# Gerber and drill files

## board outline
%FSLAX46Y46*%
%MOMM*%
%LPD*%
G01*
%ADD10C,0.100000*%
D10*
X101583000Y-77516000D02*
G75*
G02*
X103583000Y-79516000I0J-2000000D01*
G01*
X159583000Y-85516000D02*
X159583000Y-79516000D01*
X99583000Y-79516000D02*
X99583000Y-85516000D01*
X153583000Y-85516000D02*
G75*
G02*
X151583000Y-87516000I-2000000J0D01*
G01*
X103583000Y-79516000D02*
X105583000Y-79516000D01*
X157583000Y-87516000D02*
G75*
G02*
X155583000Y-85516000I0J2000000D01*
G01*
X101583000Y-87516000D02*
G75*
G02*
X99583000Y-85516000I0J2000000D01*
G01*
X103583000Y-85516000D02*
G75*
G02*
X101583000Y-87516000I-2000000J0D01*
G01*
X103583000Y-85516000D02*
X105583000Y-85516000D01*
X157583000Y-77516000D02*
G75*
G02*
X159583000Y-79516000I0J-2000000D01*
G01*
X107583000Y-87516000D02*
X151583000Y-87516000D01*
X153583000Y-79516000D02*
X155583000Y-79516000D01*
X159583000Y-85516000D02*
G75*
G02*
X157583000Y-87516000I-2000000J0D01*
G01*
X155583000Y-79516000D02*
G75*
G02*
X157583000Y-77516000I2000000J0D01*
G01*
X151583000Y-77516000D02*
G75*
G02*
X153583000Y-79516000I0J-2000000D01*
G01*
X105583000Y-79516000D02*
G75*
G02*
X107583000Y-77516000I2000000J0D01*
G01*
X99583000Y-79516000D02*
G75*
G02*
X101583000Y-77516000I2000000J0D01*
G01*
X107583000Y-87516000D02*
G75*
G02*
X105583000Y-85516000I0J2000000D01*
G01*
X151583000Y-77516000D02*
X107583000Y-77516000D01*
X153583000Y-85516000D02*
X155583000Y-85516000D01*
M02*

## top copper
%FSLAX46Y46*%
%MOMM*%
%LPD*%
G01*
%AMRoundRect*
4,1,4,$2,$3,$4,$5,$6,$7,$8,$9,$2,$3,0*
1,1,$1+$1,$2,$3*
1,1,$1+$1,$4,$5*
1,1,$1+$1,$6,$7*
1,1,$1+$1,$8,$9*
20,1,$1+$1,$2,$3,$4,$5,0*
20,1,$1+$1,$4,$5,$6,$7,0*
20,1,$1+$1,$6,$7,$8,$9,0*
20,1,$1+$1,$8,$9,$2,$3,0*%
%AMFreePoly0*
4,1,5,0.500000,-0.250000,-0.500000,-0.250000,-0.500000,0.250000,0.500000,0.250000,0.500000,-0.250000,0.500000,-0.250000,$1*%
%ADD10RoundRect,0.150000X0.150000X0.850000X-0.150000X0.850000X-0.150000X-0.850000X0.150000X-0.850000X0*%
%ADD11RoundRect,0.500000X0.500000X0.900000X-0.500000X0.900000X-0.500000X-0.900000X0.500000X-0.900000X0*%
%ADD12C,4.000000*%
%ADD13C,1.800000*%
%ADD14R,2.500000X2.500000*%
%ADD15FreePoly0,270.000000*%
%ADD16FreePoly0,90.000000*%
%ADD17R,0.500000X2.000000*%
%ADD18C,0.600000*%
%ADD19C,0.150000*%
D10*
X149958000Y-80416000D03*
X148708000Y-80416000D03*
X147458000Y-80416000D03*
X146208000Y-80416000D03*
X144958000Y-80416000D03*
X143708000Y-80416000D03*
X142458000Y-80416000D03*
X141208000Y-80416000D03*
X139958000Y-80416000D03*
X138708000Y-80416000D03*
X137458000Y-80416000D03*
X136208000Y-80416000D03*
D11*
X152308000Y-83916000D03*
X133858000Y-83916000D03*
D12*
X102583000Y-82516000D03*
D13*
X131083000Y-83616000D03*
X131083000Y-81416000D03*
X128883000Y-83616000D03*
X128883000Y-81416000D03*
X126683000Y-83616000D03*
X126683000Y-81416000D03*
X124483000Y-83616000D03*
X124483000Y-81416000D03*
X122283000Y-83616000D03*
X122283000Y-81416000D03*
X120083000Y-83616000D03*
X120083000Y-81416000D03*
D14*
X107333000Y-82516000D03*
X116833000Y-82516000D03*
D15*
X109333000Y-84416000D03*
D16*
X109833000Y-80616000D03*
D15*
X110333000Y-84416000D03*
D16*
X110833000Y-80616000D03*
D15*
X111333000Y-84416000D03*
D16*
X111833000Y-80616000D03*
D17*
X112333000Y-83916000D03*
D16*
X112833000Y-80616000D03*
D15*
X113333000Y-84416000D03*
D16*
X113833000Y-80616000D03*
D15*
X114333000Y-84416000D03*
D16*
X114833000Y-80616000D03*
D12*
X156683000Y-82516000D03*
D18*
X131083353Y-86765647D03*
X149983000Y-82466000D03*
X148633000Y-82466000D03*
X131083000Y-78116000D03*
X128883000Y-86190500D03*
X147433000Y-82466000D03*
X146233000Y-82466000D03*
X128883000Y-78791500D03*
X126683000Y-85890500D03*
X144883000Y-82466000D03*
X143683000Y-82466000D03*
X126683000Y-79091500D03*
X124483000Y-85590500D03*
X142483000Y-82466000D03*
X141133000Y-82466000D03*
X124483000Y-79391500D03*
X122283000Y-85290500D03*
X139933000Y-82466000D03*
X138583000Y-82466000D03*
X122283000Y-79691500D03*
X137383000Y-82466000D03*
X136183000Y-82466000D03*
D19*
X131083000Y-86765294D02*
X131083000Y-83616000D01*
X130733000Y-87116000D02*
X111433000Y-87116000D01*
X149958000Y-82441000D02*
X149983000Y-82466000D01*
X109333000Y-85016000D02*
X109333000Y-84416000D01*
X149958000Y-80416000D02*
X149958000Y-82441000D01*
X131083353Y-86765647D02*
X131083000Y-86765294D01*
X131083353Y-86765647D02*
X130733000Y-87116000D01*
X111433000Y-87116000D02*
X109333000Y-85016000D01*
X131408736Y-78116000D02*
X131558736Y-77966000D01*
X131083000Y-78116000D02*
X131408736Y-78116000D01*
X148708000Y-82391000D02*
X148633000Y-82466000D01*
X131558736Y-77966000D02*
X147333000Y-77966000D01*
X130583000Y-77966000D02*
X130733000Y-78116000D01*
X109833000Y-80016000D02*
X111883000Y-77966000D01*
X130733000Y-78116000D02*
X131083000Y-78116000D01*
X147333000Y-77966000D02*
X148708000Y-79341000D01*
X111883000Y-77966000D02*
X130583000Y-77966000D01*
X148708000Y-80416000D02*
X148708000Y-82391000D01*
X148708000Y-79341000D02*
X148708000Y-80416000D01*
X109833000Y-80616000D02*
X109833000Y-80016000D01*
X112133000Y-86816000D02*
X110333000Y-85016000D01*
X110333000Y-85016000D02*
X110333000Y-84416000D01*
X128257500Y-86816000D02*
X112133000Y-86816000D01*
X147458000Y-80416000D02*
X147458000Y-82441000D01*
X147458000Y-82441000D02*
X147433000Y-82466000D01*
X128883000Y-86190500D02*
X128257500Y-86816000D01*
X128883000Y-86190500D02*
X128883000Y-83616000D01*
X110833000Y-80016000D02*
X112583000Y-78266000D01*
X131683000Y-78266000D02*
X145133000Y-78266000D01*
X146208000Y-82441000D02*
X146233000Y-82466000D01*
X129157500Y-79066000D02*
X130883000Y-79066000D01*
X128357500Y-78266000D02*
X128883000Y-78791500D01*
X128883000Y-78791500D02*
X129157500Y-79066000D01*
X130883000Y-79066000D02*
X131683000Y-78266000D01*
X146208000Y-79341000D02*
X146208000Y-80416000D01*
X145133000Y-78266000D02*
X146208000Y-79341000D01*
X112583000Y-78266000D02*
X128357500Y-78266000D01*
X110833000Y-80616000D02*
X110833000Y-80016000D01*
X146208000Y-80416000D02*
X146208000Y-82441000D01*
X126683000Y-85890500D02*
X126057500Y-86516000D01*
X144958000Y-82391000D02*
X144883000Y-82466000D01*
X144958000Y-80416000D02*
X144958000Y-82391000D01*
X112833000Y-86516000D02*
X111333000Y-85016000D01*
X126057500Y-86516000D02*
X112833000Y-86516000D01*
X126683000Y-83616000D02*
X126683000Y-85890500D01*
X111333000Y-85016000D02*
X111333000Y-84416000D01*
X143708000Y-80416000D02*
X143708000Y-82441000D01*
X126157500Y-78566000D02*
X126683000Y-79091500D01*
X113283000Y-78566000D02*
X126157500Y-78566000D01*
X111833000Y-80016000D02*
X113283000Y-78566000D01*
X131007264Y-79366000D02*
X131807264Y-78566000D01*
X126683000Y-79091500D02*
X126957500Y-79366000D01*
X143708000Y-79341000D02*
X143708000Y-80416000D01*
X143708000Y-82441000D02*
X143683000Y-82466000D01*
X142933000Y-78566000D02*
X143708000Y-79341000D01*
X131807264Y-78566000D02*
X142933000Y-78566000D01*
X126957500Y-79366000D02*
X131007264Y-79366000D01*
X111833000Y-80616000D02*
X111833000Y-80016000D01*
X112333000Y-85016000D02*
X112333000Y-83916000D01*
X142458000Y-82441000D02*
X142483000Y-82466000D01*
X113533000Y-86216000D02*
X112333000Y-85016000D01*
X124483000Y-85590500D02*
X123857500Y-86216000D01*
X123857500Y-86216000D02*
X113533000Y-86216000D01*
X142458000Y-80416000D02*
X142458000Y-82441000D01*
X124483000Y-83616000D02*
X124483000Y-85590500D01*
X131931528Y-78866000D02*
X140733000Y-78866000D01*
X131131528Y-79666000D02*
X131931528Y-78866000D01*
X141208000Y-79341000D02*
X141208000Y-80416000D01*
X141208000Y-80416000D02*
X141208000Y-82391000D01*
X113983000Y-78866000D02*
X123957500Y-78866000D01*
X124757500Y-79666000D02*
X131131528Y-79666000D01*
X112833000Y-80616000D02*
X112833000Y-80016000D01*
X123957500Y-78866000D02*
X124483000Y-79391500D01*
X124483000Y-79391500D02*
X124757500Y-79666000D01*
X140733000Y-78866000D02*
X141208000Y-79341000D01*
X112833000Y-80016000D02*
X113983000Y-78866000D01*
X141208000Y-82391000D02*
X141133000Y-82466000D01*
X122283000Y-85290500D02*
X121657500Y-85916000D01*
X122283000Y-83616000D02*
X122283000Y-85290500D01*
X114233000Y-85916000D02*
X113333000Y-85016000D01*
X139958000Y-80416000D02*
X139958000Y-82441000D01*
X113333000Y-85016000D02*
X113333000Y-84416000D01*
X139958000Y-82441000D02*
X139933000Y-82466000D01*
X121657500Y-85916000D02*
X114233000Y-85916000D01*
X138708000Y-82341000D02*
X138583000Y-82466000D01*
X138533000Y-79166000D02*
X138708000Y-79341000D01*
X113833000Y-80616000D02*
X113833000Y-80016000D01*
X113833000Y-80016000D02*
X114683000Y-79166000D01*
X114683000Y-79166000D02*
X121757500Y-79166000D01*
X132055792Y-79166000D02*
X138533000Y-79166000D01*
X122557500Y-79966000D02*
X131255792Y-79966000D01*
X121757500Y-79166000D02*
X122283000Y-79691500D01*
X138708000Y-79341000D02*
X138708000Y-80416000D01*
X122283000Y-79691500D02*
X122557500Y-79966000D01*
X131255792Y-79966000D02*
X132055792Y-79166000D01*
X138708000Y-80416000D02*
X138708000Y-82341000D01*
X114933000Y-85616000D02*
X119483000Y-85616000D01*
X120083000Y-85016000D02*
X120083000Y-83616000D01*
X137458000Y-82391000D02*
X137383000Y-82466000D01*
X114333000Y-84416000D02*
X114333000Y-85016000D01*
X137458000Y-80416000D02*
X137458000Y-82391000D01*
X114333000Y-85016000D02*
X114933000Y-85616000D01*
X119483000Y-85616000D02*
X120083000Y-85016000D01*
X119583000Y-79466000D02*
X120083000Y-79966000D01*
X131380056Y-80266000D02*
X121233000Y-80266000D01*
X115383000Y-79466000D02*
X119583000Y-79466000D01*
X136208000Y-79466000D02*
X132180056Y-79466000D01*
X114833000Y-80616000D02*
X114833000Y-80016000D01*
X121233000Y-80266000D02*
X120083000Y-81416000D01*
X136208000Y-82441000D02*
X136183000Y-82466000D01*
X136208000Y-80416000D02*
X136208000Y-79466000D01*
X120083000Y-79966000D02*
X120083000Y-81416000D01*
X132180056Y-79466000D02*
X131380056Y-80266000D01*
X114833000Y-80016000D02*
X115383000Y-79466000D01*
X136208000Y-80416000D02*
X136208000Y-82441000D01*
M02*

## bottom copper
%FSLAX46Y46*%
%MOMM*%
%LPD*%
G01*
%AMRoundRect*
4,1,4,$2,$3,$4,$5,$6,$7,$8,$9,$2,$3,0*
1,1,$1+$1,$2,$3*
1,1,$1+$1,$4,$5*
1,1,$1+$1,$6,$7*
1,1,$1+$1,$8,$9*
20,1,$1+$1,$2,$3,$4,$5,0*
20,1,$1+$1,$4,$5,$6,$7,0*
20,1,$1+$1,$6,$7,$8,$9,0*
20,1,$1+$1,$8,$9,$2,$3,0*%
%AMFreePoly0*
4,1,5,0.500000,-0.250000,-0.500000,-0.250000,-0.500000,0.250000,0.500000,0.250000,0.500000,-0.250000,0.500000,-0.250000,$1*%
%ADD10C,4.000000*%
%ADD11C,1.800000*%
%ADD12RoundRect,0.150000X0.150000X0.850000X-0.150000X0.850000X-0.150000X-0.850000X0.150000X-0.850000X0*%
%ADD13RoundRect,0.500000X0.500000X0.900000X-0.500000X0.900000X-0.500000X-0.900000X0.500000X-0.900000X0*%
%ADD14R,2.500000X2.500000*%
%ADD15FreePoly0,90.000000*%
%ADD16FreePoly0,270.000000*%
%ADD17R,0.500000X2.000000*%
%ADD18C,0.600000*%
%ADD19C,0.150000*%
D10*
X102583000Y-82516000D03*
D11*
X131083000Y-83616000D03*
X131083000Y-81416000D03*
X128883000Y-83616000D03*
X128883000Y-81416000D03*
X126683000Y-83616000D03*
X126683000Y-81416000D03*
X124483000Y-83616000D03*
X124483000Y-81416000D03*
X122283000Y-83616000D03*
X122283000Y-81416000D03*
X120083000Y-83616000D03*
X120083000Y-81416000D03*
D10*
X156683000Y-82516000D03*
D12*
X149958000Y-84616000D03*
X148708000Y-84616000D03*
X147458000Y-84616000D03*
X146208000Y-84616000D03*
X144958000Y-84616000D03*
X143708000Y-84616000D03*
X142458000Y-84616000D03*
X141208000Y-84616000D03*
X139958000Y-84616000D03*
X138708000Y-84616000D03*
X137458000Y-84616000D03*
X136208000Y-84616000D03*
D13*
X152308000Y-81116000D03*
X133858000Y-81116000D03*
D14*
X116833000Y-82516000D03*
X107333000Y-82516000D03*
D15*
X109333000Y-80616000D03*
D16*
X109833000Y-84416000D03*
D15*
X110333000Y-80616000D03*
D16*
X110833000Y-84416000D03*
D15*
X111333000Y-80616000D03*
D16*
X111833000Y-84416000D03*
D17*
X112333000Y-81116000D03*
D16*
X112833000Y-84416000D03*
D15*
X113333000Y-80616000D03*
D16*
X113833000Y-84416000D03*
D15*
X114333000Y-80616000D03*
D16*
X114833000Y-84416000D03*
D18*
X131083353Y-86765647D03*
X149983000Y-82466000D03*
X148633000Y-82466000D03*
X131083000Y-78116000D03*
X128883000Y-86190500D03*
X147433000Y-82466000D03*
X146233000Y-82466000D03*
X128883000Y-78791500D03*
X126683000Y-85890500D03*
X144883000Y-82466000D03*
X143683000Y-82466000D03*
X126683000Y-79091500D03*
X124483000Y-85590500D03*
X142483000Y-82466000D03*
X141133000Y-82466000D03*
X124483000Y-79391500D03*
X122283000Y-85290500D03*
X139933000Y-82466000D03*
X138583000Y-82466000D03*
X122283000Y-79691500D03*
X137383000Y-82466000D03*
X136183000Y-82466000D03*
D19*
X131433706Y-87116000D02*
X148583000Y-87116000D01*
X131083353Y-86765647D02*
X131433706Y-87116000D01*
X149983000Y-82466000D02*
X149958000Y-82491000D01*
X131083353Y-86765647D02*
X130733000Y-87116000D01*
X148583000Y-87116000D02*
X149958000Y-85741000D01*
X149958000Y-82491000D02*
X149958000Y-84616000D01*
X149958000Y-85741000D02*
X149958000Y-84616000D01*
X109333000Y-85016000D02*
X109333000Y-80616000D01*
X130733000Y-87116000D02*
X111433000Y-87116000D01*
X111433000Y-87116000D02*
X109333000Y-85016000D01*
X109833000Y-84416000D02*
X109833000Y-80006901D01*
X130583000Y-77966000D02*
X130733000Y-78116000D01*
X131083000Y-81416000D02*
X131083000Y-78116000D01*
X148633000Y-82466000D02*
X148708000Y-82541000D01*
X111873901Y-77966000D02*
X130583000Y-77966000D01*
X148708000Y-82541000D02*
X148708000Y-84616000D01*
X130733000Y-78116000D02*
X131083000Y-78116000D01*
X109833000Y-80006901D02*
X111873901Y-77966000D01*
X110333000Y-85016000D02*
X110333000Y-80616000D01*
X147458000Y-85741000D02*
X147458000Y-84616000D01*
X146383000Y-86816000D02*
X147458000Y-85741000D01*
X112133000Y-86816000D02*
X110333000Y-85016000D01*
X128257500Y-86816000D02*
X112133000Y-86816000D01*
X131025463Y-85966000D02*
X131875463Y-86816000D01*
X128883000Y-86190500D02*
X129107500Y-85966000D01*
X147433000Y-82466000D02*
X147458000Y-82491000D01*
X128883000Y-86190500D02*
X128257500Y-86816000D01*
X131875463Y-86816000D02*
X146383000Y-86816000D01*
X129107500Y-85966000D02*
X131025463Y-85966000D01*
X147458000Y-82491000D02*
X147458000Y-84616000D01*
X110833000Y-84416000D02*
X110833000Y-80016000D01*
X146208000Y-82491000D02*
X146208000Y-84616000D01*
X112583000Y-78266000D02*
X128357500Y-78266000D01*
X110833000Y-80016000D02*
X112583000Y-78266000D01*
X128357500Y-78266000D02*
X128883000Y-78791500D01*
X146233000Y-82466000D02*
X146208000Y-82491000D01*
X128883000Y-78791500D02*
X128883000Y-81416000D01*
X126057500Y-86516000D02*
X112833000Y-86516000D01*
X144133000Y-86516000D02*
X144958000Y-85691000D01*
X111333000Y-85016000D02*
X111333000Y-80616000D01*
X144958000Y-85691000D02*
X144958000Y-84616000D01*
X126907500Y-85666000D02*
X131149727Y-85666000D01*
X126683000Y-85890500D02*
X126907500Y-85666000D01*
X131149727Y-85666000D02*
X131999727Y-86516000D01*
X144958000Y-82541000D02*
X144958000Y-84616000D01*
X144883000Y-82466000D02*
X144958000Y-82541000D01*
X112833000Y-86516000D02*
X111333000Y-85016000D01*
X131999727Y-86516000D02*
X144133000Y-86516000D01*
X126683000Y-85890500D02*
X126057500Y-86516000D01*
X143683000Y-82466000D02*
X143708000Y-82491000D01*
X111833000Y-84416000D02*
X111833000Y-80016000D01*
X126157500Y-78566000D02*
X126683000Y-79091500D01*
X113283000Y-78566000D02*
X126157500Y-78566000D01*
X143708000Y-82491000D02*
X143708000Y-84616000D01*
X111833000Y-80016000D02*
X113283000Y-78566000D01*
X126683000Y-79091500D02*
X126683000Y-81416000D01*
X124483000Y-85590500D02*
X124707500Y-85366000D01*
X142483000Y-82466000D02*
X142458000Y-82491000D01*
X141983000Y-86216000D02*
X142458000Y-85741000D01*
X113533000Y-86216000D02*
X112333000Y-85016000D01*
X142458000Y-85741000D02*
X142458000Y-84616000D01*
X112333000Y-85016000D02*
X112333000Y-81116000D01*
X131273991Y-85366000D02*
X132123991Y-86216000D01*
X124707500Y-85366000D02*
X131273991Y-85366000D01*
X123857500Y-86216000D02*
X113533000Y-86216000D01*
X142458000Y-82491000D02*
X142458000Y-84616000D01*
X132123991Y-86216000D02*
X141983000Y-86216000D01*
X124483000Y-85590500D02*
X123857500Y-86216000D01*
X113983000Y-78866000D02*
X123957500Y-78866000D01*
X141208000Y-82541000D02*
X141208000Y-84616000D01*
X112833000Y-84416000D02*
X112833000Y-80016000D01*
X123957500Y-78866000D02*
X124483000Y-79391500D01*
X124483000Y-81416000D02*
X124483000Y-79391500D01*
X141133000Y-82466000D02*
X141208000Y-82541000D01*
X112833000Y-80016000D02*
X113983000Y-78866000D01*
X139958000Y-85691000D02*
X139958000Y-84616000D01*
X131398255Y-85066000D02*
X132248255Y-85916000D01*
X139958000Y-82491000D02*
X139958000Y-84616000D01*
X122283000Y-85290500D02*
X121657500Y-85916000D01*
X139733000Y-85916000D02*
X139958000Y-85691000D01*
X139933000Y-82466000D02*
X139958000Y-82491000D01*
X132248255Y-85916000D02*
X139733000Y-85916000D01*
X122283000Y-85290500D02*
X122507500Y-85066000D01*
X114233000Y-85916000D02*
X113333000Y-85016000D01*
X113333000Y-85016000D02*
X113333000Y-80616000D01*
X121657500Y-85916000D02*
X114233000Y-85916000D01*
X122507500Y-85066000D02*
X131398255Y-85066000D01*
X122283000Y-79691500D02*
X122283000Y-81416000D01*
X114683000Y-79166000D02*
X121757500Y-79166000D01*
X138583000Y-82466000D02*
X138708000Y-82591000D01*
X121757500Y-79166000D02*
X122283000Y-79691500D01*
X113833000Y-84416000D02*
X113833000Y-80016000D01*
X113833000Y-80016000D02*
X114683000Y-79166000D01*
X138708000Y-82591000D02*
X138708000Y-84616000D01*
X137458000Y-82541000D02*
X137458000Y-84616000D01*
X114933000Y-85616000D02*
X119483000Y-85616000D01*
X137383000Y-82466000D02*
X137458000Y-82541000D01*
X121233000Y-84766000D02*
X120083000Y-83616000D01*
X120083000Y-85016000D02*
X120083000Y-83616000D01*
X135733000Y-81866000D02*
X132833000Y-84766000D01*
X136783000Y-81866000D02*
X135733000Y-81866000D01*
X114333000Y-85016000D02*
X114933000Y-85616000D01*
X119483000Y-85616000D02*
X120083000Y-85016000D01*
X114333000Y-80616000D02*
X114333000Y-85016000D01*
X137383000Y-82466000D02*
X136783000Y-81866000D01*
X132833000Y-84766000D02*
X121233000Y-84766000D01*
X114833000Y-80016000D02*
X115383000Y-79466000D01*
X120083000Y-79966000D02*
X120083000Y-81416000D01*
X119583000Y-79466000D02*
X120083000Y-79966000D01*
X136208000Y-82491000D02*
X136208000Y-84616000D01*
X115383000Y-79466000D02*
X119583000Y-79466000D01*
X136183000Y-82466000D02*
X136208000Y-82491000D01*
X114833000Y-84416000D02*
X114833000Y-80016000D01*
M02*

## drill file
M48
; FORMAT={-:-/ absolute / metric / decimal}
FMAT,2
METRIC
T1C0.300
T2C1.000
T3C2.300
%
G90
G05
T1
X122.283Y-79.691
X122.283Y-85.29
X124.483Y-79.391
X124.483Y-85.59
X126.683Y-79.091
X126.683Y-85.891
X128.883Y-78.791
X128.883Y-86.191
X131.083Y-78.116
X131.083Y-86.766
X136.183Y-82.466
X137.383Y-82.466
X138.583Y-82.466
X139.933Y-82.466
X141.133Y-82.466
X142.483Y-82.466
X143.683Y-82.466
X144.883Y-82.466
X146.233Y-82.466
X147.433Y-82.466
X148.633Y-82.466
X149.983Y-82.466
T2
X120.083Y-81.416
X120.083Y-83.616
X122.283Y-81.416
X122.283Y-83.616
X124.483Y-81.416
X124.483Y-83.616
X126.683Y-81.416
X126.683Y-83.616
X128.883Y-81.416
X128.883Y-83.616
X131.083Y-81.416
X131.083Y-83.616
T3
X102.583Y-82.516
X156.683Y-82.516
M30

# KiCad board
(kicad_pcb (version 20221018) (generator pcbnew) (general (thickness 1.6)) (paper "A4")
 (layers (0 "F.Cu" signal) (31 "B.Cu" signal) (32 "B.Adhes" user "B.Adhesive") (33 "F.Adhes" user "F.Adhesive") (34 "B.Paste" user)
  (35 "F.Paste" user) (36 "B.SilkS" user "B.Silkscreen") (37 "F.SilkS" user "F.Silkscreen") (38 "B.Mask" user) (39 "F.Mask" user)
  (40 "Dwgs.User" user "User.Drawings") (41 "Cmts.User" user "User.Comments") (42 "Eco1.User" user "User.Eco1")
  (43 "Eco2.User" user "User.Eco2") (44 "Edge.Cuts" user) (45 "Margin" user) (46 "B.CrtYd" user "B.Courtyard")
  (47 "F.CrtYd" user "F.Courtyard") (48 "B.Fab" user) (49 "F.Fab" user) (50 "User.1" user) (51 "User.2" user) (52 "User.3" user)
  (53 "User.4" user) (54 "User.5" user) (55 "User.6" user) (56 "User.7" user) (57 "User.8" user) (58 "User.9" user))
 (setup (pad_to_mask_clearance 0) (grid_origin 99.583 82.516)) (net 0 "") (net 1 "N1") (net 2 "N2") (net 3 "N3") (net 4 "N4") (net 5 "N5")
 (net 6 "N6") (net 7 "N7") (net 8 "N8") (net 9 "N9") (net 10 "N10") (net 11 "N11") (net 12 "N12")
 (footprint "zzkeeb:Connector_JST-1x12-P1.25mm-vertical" (layer "F.Cu") (at 143.083 82.516 180)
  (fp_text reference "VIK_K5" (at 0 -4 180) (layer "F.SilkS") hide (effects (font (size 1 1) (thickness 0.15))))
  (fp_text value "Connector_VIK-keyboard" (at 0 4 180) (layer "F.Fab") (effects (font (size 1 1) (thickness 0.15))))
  (pad "1" smd roundrect (at -6.875 2.1 180) (size 0.6 2) (layers "F.Cu" "F.Paste" "F.Mask") (roundrect_rratio 0.25) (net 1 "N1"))
  (pad "2" smd roundrect (at -5.625 2.1 180) (size 0.6 2) (layers "F.Cu" "F.Paste" "F.Mask") (roundrect_rratio 0.25) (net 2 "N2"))
  (pad "3" smd roundrect (at -4.375 2.1 180) (size 0.6 2) (layers "F.Cu" "F.Paste" "F.Mask") (roundrect_rratio 0.25) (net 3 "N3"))
  (pad "4" smd roundrect (at -3.125 2.1 180) (size 0.6 2) (layers "F.Cu" "F.Paste" "F.Mask") (roundrect_rratio 0.25) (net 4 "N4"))
  (pad "5" smd roundrect (at -1.875 2.1 180) (size 0.6 2) (layers "F.Cu" "F.Paste" "F.Mask") (roundrect_rratio 0.25) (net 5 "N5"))
  (pad "6" smd roundrect (at -0.625 2.1 180) (size 0.6 2) (layers "F.Cu" "F.Paste" "F.Mask") (roundrect_rratio 0.25) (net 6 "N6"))
  (pad "7" smd roundrect (at 0.625 2.1 180) (size 0.6 2) (layers "F.Cu" "F.Paste" "F.Mask") (roundrect_rratio 0.25) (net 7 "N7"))
  (pad "8" smd roundrect (at 1.875 2.1 180) (size 0.6 2) (layers "F.Cu" "F.Paste" "F.Mask") (roundrect_rratio 0.25) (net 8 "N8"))
  (pad "9" smd roundrect (at 3.125 2.1 180) (size 0.6 2) (layers "F.Cu" "F.Paste" "F.Mask") (roundrect_rratio 0.25) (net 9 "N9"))
  (pad "10" smd roundrect (at 4.375 2.1 180) (size 0.6 2) (layers "F.Cu" "F.Paste" "F.Mask") (roundrect_rratio 0.25) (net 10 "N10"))
  (pad "11" smd roundrect (at 5.625 2.1 180) (size 0.6 2) (layers "F.Cu" "F.Paste" "F.Mask") (roundrect_rratio 0.25) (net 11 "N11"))
  (pad "12" smd roundrect (at 6.875 2.1 180) (size 0.6 2) (layers "F.Cu" "F.Paste" "F.Mask") (roundrect_rratio 0.25) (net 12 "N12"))
  (pad "MP" smd roundrect (at -9.225 -1.4 180) (size 2 2.8) (layers "F.Cu" "F.Paste" "F.Mask") (roundrect_rratio 0.25))
  (pad "MP" smd roundrect (at 9.225 -1.4 180) (size 2 2.8) (layers "F.Cu" "F.Paste" "F.Mask") (roundrect_rratio 0.25)))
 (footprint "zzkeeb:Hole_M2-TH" (layer "F.Cu") (at 102.583 82.516)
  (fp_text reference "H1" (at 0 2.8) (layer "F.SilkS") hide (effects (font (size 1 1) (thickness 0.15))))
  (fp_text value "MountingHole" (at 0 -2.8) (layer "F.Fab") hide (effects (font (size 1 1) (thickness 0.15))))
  (pad "" thru_hole circle (at 0 0) (size 4 4) (drill 2.3) (layers "*.Cu" "*.Mask")))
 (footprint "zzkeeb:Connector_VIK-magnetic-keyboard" (layer "F.Cu") (at 125.583 82.516 90)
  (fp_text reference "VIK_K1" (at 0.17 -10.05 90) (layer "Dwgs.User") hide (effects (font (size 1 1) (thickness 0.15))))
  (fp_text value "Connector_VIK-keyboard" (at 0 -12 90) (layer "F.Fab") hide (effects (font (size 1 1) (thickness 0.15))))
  (pad "1" thru_hole circle (at -1.1 5.5 270) (size 1.8 1.8) (drill 1) (layers "*.Cu" "*.Mask") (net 1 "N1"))
  (pad "2" thru_hole circle (at 1.1 5.5 270) (size 1.8 1.8) (drill 1) (layers "*.Cu" "*.Mask") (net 2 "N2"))
  (pad "3" thru_hole circle (at -1.1 3.3 270) (size 1.8 1.8) (drill 1) (layers "*.Cu" "*.Mask") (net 3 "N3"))
  (pad "4" thru_hole circle (at 1.1 3.3 270) (size 1.8 1.8) (drill 1) (layers "*.Cu" "*.Mask") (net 4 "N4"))
  (pad "5" thru_hole circle (at -1.1 1.1 270) (size 1.8 1.8) (drill 1) (layers "*.Cu" "*.Mask") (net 5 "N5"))
  (pad "6" thru_hole circle (at 1.1 1.1 270) (size 1.8 1.8) (drill 1) (layers "*.Cu" "*.Mask") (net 6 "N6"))
  (pad "7" thru_hole circle (at -1.1 -1.1 270) (size 1.8 1.8) (drill 1) (layers "*.Cu" "*.Mask") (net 7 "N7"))
  (pad "8" thru_hole circle (at 1.1 -1.1 270) (size 1.8 1.8) (drill 1) (layers "*.Cu" "*.Mask") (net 8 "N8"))
  (pad "9" thru_hole circle (at -1.1 -3.3 270) (size 1.8 1.8) (drill 1) (layers "*.Cu" "*.Mask") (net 9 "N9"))
  (pad "10" thru_hole circle (at 1.1 -3.3 270) (size 1.8 1.8) (drill 1) (layers "*.Cu" "*.Mask") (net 10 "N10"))
  (pad "11" thru_hole circle (at -1.1 -5.5 270) (size 1.8 1.8) (drill 1) (layers "*.Cu" "*.Mask") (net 11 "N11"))
  (pad "12" thru_hole circle (at 1.1 -5.5 270) (size 1.8 1.8) (drill 1) (layers "*.Cu" "*.Mask") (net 12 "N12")))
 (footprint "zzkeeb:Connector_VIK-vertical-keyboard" (layer "F.Cu") (at 112.083 82.516 90)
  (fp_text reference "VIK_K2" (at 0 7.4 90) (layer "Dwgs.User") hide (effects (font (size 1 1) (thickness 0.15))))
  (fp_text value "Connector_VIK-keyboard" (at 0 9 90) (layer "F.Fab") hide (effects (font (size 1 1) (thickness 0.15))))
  (pad "" smd rect (at 0 -4.75 90) (size 2.5 2.5) (layers "F.Cu" "F.Paste" "F.Mask"))
  (pad "" smd rect (at 0 4.75 90) (size 2.5 2.5) (layers "F.Cu" "F.Paste" "F.Mask"))
  (pad "1" smd custom (at -1.9 -2.75 270) (size 1 0.5) (layers "F.Cu" "F.Paste" "F.Mask") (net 1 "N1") (thermal_bridge_angle 45)
   (options (clearance outline) (anchor rect)) (primitives))
  (pad "2" smd custom (at 1.9 -2.25 90) (size 1 0.5) (layers "F.Cu" "F.Paste" "F.Mask") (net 2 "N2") (thermal_bridge_angle 45)
   (options (clearance outline) (anchor rect)) (primitives))
  (pad "3" smd custom (at -1.9 -1.75 270) (size 1 0.5) (layers "F.Cu" "F.Paste" "F.Mask") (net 3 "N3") (thermal_bridge_angle 45)
   (options (clearance outline) (anchor rect)) (primitives))
  (pad "4" smd custom (at 1.9 -1.25 90) (size 1 0.5) (layers "F.Cu" "F.Paste" "F.Mask") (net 4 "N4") (thermal_bridge_angle 45)
   (options (clearance outline) (anchor rect)) (primitives))
  (pad "5" smd custom (at -1.9 -0.75 270) (size 1 0.5) (layers "F.Cu" "F.Paste" "F.Mask") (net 5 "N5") (thermal_bridge_angle 45)
   (options (clearance outline) (anchor rect)) (primitives))
  (pad "6" smd custom (at 1.9 -0.25 90) (size 1 0.5) (layers "F.Cu" "F.Paste" "F.Mask") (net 6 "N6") (thermal_bridge_angle 45)
   (options (clearance outline) (anchor rect)) (primitives))
  (pad "7" smd rect (at -1.4 0.25) (size 0.5 2) (layers "F.Cu" "F.Paste" "F.Mask") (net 7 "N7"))
  (pad "8" smd custom (at 1.9 0.75 90) (size 1 0.5) (layers "F.Cu" "F.Paste" "F.Mask") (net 8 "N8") (thermal_bridge_angle 45)
   (options (clearance outline) (anchor rect)) (primitives))
  (pad "9" smd custom (at -1.9 1.25 270) (size 1 0.5) (layers "F.Cu" "F.Paste" "F.Mask") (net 9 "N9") (thermal_bridge_angle 45)
   (options (clearance outline) (anchor rect)) (primitives))
  (pad "10" smd custom (at 1.9 1.75 90) (size 1 0.5) (layers "F.Cu" "F.Paste" "F.Mask") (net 10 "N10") (thermal_bridge_angle 45)
   (options (clearance outline) (anchor rect)) (primitives))
  (pad "11" smd custom (at -1.9 2.25 270) (size 1 0.5) (layers "F.Cu" "F.Paste" "F.Mask") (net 11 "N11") (thermal_bridge_angle 45)
   (options (clearance outline) (anchor rect)) (primitives))
  (pad "12" smd custom (at 1.9 2.75 90) (size 1 0.5) (layers "F.Cu" "F.Paste" "F.Mask") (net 12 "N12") (thermal_bridge_angle 45)
   (options (clearance outline) (anchor rect)) (primitives)))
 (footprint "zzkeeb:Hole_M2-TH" (layer "F.Cu") (at 156.683 82.516)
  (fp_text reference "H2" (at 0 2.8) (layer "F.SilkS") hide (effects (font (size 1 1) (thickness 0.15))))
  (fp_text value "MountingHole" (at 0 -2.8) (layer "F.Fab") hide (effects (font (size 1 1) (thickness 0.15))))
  (pad "" thru_hole circle (at 0 0) (size 4 4) (drill 2.3) (layers "*.Cu" "*.Mask")))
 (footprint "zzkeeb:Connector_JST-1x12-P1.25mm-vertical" (layer "B.Cu") (at 143.083 82.516 180)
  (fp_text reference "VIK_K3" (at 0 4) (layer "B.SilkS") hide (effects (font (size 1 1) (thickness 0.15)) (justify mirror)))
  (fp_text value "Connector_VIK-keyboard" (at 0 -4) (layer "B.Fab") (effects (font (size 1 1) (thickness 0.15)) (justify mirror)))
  (pad "1" smd roundrect (at -6.875 -2.1 180) (size 0.6 2) (layers "B.Cu" "B.Paste" "B.Mask") (roundrect_rratio 0.25) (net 1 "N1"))
  (pad "2" smd roundrect (at -5.625 -2.1 180) (size 0.6 2) (layers "B.Cu" "B.Paste" "B.Mask") (roundrect_rratio 0.25) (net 2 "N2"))
  (pad "3" smd roundrect (at -4.375 -2.1 180) (size 0.6 2) (layers "B.Cu" "B.Paste" "B.Mask") (roundrect_rratio 0.25) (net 3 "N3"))
  (pad "4" smd roundrect (at -3.125 -2.1 180) (size 0.6 2) (layers "B.Cu" "B.Paste" "B.Mask") (roundrect_rratio 0.25) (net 4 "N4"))
  (pad "5" smd roundrect (at -1.875 -2.1 180) (size 0.6 2) (layers "B.Cu" "B.Paste" "B.Mask") (roundrect_rratio 0.25) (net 5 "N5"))
  (pad "6" smd roundrect (at -0.625 -2.1 180) (size 0.6 2) (layers "B.Cu" "B.Paste" "B.Mask") (roundrect_rratio 0.25) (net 6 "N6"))
  (pad "7" smd roundrect (at 0.625 -2.1 180) (size 0.6 2) (layers "B.Cu" "B.Paste" "B.Mask") (roundrect_rratio 0.25) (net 7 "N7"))
  (pad "8" smd roundrect (at 1.875 -2.1 180) (size 0.6 2) (layers "B.Cu" "B.Paste" "B.Mask") (roundrect_rratio 0.25) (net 8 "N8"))
  (pad "9" smd roundrect (at 3.125 -2.1 180) (size 0.6 2) (layers "B.Cu" "B.Paste" "B.Mask") (roundrect_rratio 0.25) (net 9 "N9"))
  (pad "10" smd roundrect (at 4.375 -2.1 180) (size 0.6 2) (layers "B.Cu" "B.Paste" "B.Mask") (roundrect_rratio 0.25) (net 10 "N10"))
  (pad "11" smd roundrect (at 5.625 -2.1 180) (size 0.6 2) (layers "B.Cu" "B.Paste" "B.Mask") (roundrect_rratio 0.25) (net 11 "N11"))
  (pad "12" smd roundrect (at 6.875 -2.1 180) (size 0.6 2) (layers "B.Cu" "B.Paste" "B.Mask") (roundrect_rratio 0.25) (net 12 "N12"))
  (pad "MP" smd roundrect (at -9.225 1.4 180) (size 2 2.8) (layers "B.Cu" "B.Paste" "B.Mask") (roundrect_rratio 0.25))
  (pad "MP" smd roundrect (at 9.225 1.4 180) (size 2 2.8) (layers "B.Cu" "B.Paste" "B.Mask") (roundrect_rratio 0.25)))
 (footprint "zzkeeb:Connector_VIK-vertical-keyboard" (layer "B.Cu") (at 112.083 82.516 -90)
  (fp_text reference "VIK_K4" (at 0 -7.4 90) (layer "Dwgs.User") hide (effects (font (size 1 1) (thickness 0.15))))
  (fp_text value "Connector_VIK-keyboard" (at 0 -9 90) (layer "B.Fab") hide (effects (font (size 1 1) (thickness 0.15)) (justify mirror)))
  (pad "" smd rect (at 0 -4.75 270) (size 2.5 2.5) (layers "B.Cu" "B.Paste" "B.Mask"))
  (pad "" smd rect (at 0 4.75 270) (size 2.5 2.5) (layers "B.Cu" "B.Paste" "B.Mask"))
  (pad "1" smd custom (at -1.9 2.75 90) (size 1 0.5) (layers "B.Cu" "B.Paste" "B.Mask") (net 1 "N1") (thermal_bridge_angle 45)
   (options (clearance outline) (anchor rect)) (primitives))
  (pad "2" smd custom (at 1.9 2.25 270) (size 1 0.5) (layers "B.Cu" "B.Paste" "B.Mask") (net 2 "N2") (thermal_bridge_angle 45)
   (options (clearance outline) (anchor rect)) (primitives))
  (pad "3" smd custom (at -1.9 1.75 90) (size 1 0.5) (layers "B.Cu" "B.Paste" "B.Mask") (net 3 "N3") (thermal_bridge_angle 45)
   (options (clearance outline) (anchor rect)) (primitives))
  (pad "4" smd custom (at 1.9 1.25 270) (size 1 0.5) (layers "B.Cu" "B.Paste" "B.Mask") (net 4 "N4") (thermal_bridge_angle 45)
   (options (clearance outline) (anchor rect)) (primitives))
  (pad "5" smd custom (at -1.9 0.75 90) (size 1 0.5) (layers "B.Cu" "B.Paste" "B.Mask") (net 5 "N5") (thermal_bridge_angle 45)
   (options (clearance outline) (anchor rect)) (primitives))
  (pad "6" smd custom (at 1.9 0.25 270) (size 1 0.5) (layers "B.Cu" "B.Paste" "B.Mask") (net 6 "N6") (thermal_bridge_angle 45)
   (options (clearance outline) (anchor rect)) (primitives))
  (pad "7" smd rect (at -1.4 -0.25) (size 0.5 2) (layers "B.Cu" "B.Paste" "B.Mask") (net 7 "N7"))
  (pad "8" smd custom (at 1.9 -0.75 270) (size 1 0.5) (layers "B.Cu" "B.Paste" "B.Mask") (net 8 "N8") (thermal_bridge_angle 45)
   (options (clearance outline) (anchor rect)) (primitives))
  (pad "9" smd custom (at -1.9 -1.25 90) (size 1 0.5) (layers "B.Cu" "B.Paste" "B.Mask") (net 9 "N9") (thermal_bridge_angle 45)
   (options (clearance outline) (anchor rect)) (primitives))
  (pad "10" smd custom (at 1.9 -1.75 270) (size 1 0.5) (layers "B.Cu" "B.Paste" "B.Mask") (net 10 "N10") (thermal_bridge_angle 45)
   (options (clearance outline) (anchor rect)) (primitives))
  (pad "11" smd custom (at -1.9 -2.25 90) (size 1 0.5) (layers "B.Cu" "B.Paste" "B.Mask") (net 11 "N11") (thermal_bridge_angle 45)
   (options (clearance outline) (anchor rect)) (primitives))
  (pad "12" smd custom (at 1.9 -2.75 270) (size 1 0.5) (layers "B.Cu" "B.Paste" "B.Mask") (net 12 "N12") (thermal_bridge_angle 45)
   (options (clearance outline) (anchor rect)) (primitives)))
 (gr_arc (start 101.583 77.516) (mid 102.997214 78.101786) (end 103.583 79.516) (stroke (width 0.1) (type default)) (layer "Edge.Cuts"))
 (gr_line (start 159.583 85.516) (end 159.583 79.516) (stroke (width 0.1) (type default)) (layer "Edge.Cuts"))
 (gr_line (start 99.583 79.516) (end 99.583 85.516) (stroke (width 0.1) (type default)) (layer "Edge.Cuts"))
 (gr_arc (start 153.583 85.516) (mid 152.997214 86.930214) (end 151.583 87.516) (stroke (width 0.1) (type default)) (layer "Edge.Cuts"))
 (gr_line (start 103.583 79.516) (end 105.583 79.516) (stroke (width 0.1) (type default)) (layer "Edge.Cuts"))
 (gr_arc (start 157.583 87.516) (mid 156.168786 86.930214) (end 155.583 85.516) (stroke (width 0.1) (type default)) (layer "Edge.Cuts"))
 (gr_arc (start 101.583 87.516) (mid 100.168786 86.930214) (end 99.583 85.516) (stroke (width 0.1) (type default)) (layer "Edge.Cuts"))
 (gr_arc (start 103.583 85.516) (mid 102.997214 86.930214) (end 101.583 87.516) (stroke (width 0.1) (type default)) (layer "Edge.Cuts"))
 (gr_line (start 103.583 85.516) (end 105.583 85.516) (stroke (width 0.1) (type default)) (layer "Edge.Cuts"))
 (gr_arc (start 157.583 77.516) (mid 158.997214 78.101786) (end 159.583 79.516) (stroke (width 0.1) (type default)) (layer "Edge.Cuts"))
 (gr_line (start 107.583 87.516) (end 151.583 87.516) (stroke (width 0.1) (type default)) (layer "Edge.Cuts"))
 (gr_line (start 153.583 79.516) (end 155.583 79.516) (stroke (width 0.1) (type default)) (layer "Edge.Cuts"))
 (gr_arc (start 159.583 85.516) (mid 158.997214 86.930214) (end 157.583 87.516) (stroke (width 0.1) (type default)) (layer "Edge.Cuts"))
 (gr_arc (start 155.583 79.516) (mid 156.168786 78.101786) (end 157.583 77.516) (stroke (width 0.1) (type default)) (layer "Edge.Cuts"))
 (gr_arc (start 151.583 77.516) (mid 152.997214 78.101786) (end 153.583 79.516) (stroke (width 0.1) (type default)) (layer "Edge.Cuts"))
 (gr_arc (start 105.583 79.516) (mid 106.168786 78.101786) (end 107.583 77.516) (stroke (width 0.1) (type default)) (layer "Edge.Cuts"))
 (gr_arc (start 99.583 79.516) (mid 100.168786 78.101786) (end 101.583 77.516) (stroke (width 0.1) (type default)) (layer "Edge.Cuts"))
 (gr_arc (start 107.583 87.516) (mid 106.168786 86.930214) (end 105.583 85.516) (stroke (width 0.1) (type default)) (layer "Edge.Cuts"))
 (gr_line (start 151.583 77.516) (end 107.583 77.516) (stroke (width 0.1) (type default)) (layer "Edge.Cuts"))
 (gr_line (start 153.583 85.516) (end 155.583 85.516) (stroke (width 0.1) (type default)) (layer "Edge.Cuts"))
 (segment (start 131.083 86.765294) (end 131.083 83.616) (width 0.15) (layer "F.Cu") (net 1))
 (segment (start 130.733 87.116) (end 111.433 87.116) (width 0.15) (layer "F.Cu") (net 1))
 (segment (start 149.958 82.441) (end 149.983 82.466) (width 0.15) (layer "F.Cu") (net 1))
 (segment (start 109.333 85.016) (end 109.333 84.416) (width 0.15) (layer "F.Cu") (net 1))
 (segment (start 149.958 80.416) (end 149.958 82.441) (width 0.15) (layer "F.Cu") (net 1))
 (segment (start 131.083353 86.765647) (end 131.083 86.765294) (width 0.15) (layer "F.Cu") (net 1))
 (segment (start 131.083353 86.765647) (end 130.733 87.116) (width 0.15) (layer "F.Cu") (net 1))
 (segment (start 111.433 87.116) (end 109.333 85.016) (width 0.15) (layer "F.Cu") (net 1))
 (via (at 131.083353 86.765647) (size 0.6) (drill 0.3) (layers "F.Cu" "B.Cu") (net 1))
 (via (at 149.983 82.466) (size 0.6) (drill 0.3) (layers "F.Cu" "B.Cu") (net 1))
 (segment (start 131.433706 87.116) (end 148.583 87.116) (width 0.15) (layer "B.Cu") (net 1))
 (segment (start 131.083353 86.765647) (end 131.433706 87.116) (width 0.15) (layer "B.Cu") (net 1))
 (segment (start 149.983 82.466) (end 149.958 82.491) (width 0.15) (layer "B.Cu") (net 1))
 (segment (start 131.083353 86.765647) (end 130.733 87.116) (width 0.15) (layer "B.Cu") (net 1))
 (segment (start 148.583 87.116) (end 149.958 85.741) (width 0.15) (layer "B.Cu") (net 1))
 (segment (start 149.958 82.491) (end 149.958 84.616) (width 0.15) (layer "B.Cu") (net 1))
 (segment (start 149.958 85.741) (end 149.958 84.616) (width 0.15) (layer "B.Cu") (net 1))
 (segment (start 109.333 85.016) (end 109.333 80.616) (width 0.15) (layer "B.Cu") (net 1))
 (segment (start 130.733 87.116) (end 111.433 87.116) (width 0.15) (layer "B.Cu") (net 1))
 (segment (start 111.433 87.116) (end 109.333 85.016) (width 0.15) (layer "B.Cu") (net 1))
 (segment (start 131.408736 78.116) (end 131.558736 77.966) (width 0.15) (layer "F.Cu") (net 2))
 (segment (start 131.083 78.116) (end 131.408736 78.116) (width 0.15) (layer "F.Cu") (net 2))
 (segment (start 148.708 82.391) (end 148.633 82.466) (width 0.15) (layer "F.Cu") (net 2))
 (segment (start 131.558736 77.966) (end 147.333 77.966) (width 0.15) (layer "F.Cu") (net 2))
 (segment (start 130.583 77.966) (end 130.733 78.116) (width 0.15) (layer "F.Cu") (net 2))
 (segment (start 109.833 80.016) (end 111.883 77.966) (width 0.15) (layer "F.Cu") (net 2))
 (segment (start 130.733 78.116) (end 131.083 78.116) (width 0.15) (layer "F.Cu") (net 2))
 (segment (start 147.333 77.966) (end 148.708 79.341) (width 0.15) (layer "F.Cu") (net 2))
 (segment (start 111.883 77.966) (end 130.583 77.966) (width 0.15) (layer "F.Cu") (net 2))
 (segment (start 148.708 80.416) (end 148.708 82.391) (width 0.15) (layer "F.Cu") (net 2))
 (segment (start 148.708 79.341) (end 148.708 80.416) (width 0.15) (layer "F.Cu") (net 2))
 (segment (start 109.833 80.616) (end 109.833 80.016) (width 0.15) (layer "F.Cu") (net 2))
 (via (at 148.633 82.466) (size 0.6) (drill 0.3) (layers "F.Cu" "B.Cu") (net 2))
 (via (at 131.083 78.116) (size 0.6) (drill 0.3) (layers "F.Cu" "B.Cu") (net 2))
 (segment (start 109.833 84.416) (end 109.833 80.006901) (width 0.15) (layer "B.Cu") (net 2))
 (segment (start 130.583 77.966) (end 130.733 78.116) (width 0.15) (layer "B.Cu") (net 2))
 (segment (start 131.083 81.416) (end 131.083 78.116) (width 0.15) (layer "B.Cu") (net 2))
 (segment (start 148.633 82.466) (end 148.708 82.541) (width 0.15) (layer "B.Cu") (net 2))
 (segment (start 111.873901 77.966) (end 130.583 77.966) (width 0.15) (layer "B.Cu") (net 2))
 (segment (start 148.708 82.541) (end 148.708 84.616) (width 0.15) (layer "B.Cu") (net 2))
 (segment (start 130.733 78.116) (end 131.083 78.116) (width 0.15) (layer "B.Cu") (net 2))
 (segment (start 109.833 80.006901) (end 111.873901 77.966) (width 0.15) (layer "B.Cu") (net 2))
 (segment (start 112.133 86.816) (end 110.333 85.016) (width 0.15) (layer "F.Cu") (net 3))
 (segment (start 110.333 85.016) (end 110.333 84.416) (width 0.15) (layer "F.Cu") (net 3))
 (segment (start 128.2575 86.816) (end 112.133 86.816) (width 0.15) (layer "F.Cu") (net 3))
 (segment (start 147.458 80.416) (end 147.458 82.441) (width 0.15) (layer "F.Cu") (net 3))
 (segment (start 147.458 82.441) (end 147.433 82.466) (width 0.15) (layer "F.Cu") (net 3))
 (segment (start 128.883 86.1905) (end 128.2575 86.816) (width 0.15) (layer "F.Cu") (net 3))
 (segment (start 128.883 86.1905) (end 128.883 83.616) (width 0.15) (layer "F.Cu") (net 3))
 (via (at 128.883 86.1905) (size 0.6) (drill 0.3) (layers "F.Cu" "B.Cu") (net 3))
 (via (at 147.433 82.466) (size 0.6) (drill 0.3) (layers "F.Cu" "B.Cu") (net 3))
 (segment (start 110.333 85.016) (end 110.333 80.616) (width 0.15) (layer "B.Cu") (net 3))
 (segment (start 147.458 85.741) (end 147.458 84.616) (width 0.15) (layer "B.Cu") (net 3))
 (segment (start 146.383 86.816) (end 147.458 85.741) (width 0.15) (layer "B.Cu") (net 3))
 (segment (start 112.133 86.816) (end 110.333 85.016) (width 0.15) (layer "B.Cu") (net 3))
 (segment (start 128.2575 86.816) (end 112.133 86.816) (width 0.15) (layer "B.Cu") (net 3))
 (segment (start 131.025463 85.966) (end 131.875463 86.816) (width 0.15) (layer "B.Cu") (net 3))
 (segment (start 128.883 86.1905) (end 129.1075 85.966) (width 0.15) (layer "B.Cu") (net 3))
 (segment (start 147.433 82.466) (end 147.458 82.491) (width 0.15) (layer "B.Cu") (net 3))
 (segment (start 128.883 86.1905) (end 128.2575 86.816) (width 0.15) (layer "B.Cu") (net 3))
 (segment (start 131.875463 86.816) (end 146.383 86.816) (width 0.15) (layer "B.Cu") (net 3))
 (segment (start 129.1075 85.966) (end 131.025463 85.966) (width 0.15) (layer "B.Cu") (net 3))
 (segment (start 147.458 82.491) (end 147.458 84.616) (width 0.15) (layer "B.Cu") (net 3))
 (segment (start 110.833 80.016) (end 112.583 78.266) (width 0.15) (layer "F.Cu") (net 4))
 (segment (start 131.683 78.266) (end 145.133 78.266) (width 0.15) (layer "F.Cu") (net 4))
 (segment (start 146.208 82.441) (end 146.233 82.466) (width 0.15) (layer "F.Cu") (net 4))
 (segment (start 129.1575 79.066) (end 130.883 79.066) (width 0.15) (layer "F.Cu") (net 4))
 (segment (start 128.3575 78.266) (end 128.883 78.7915) (width 0.15) (layer "F.Cu") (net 4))
 (segment (start 128.883 78.7915) (end 129.1575 79.066) (width 0.15) (layer "F.Cu") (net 4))
 (segment (start 130.883 79.066) (end 131.683 78.266) (width 0.15) (layer "F.Cu") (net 4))
 (segment (start 146.208 79.341) (end 146.208 80.416) (width 0.15) (layer "F.Cu") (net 4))
 (segment (start 145.133 78.266) (end 146.208 79.341) (width 0.15) (layer "F.Cu") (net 4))
 (segment (start 112.583 78.266) (end 128.3575 78.266) (width 0.15) (layer "F.Cu") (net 4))
 (segment (start 110.833 80.616) (end 110.833 80.016) (width 0.15) (layer "F.Cu") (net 4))
 (segment (start 146.208 80.416) (end 146.208 82.441) (width 0.15) (layer "F.Cu") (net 4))
 (via (at 146.233 82.466) (size 0.6) (drill 0.3) (layers "F.Cu" "B.Cu") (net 4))
 (via (at 128.883 78.7915) (size 0.6) (drill 0.3) (layers "F.Cu" "B.Cu") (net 4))
 (segment (start 110.833 84.416) (end 110.833 80.016) (width 0.15) (layer "B.Cu") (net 4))
 (segment (start 146.208 82.491) (end 146.208 84.616) (width 0.15) (layer "B.Cu") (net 4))
 (segment (start 112.583 78.266) (end 128.3575 78.266) (width 0.15) (layer "B.Cu") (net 4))
 (segment (start 110.833 80.016) (end 112.583 78.266) (width 0.15) (layer "B.Cu") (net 4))
 (segment (start 128.3575 78.266) (end 128.883 78.7915) (width 0.15) (layer "B.Cu") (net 4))
 (segment (start 146.233 82.466) (end 146.208 82.491) (width 0.15) (layer "B.Cu") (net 4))
 (segment (start 128.883 78.7915) (end 128.883 81.416) (width 0.15) (layer "B.Cu") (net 4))
 (segment (start 126.683 85.8905) (end 126.0575 86.516) (width 0.15) (layer "F.Cu") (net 5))
 (segment (start 144.958 82.391) (end 144.883 82.466) (width 0.15) (layer "F.Cu") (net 5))
 (segment (start 144.958 80.416) (end 144.958 82.391) (width 0.15) (layer "F.Cu") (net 5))
 (segment (start 112.833 86.516) (end 111.333 85.016) (width 0.15) (layer "F.Cu") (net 5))
 (segment (start 126.0575 86.516) (end 112.833 86.516) (width 0.15) (layer "F.Cu") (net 5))
 (segment (start 126.683 83.616) (end 126.683 85.8905) (width 0.15) (layer "F.Cu") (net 5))
 (segment (start 111.333 85.016) (end 111.333 84.416) (width 0.15) (layer "F.Cu") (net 5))
 (via (at 126.683 85.8905) (size 0.6) (drill 0.3) (layers "F.Cu" "B.Cu") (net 5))
 (via (at 144.883 82.466) (size 0.6) (drill 0.3) (layers "F.Cu" "B.Cu") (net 5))
 (segment (start 126.0575 86.516) (end 112.833 86.516) (width 0.15) (layer "B.Cu") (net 5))
 (segment (start 144.133 86.516) (end 144.958 85.691) (width 0.15) (layer "B.Cu") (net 5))
 (segment (start 111.333 85.016) (end 111.333 80.616) (width 0.15) (layer "B.Cu") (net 5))
 (segment (start 144.958 85.691) (end 144.958 84.616) (width 0.15) (layer "B.Cu") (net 5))
 (segment (start 126.9075 85.666) (end 131.149727 85.666) (width 0.15) (layer "B.Cu") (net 5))
 (segment (start 126.683 85.8905) (end 126.9075 85.666) (width 0.15) (layer "B.Cu") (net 5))
 (segment (start 131.149727 85.666) (end 131.999727 86.516) (width 0.15) (layer "B.Cu") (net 5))
 (segment (start 144.958 82.541) (end 144.958 84.616) (width 0.15) (layer "B.Cu") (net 5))
 (segment (start 144.883 82.466) (end 144.958 82.541) (width 0.15) (layer "B.Cu") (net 5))
 (segment (start 112.833 86.516) (end 111.333 85.016) (width 0.15) (layer "B.Cu") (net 5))
 (segment (start 131.999727 86.516) (end 144.133 86.516) (width 0.15) (layer "B.Cu") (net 5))
 (segment (start 126.683 85.8905) (end 126.0575 86.516) (width 0.15) (layer "B.Cu") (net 5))
 (segment (start 143.708 80.416) (end 143.708 82.441) (width 0.15) (layer "F.Cu") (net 6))
 (segment (start 126.1575 78.566) (end 126.683 79.0915) (width 0.15) (layer "F.Cu") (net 6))
 (segment (start 113.283 78.566) (end 126.1575 78.566) (width 0.15) (layer "F.Cu") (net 6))
 (segment (start 111.833 80.016) (end 113.283 78.566) (width 0.15) (layer "F.Cu") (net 6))
 (segment (start 131.007264 79.366) (end 131.807264 78.566) (width 0.15) (layer "F.Cu") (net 6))
 (segment (start 126.683 79.0915) (end 126.9575 79.366) (width 0.15) (layer "F.Cu") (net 6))
 (segment (start 143.708 79.341) (end 143.708 80.416) (width 0.15) (layer "F.Cu") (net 6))
 (segment (start 143.708 82.441) (end 143.683 82.466) (width 0.15) (layer "F.Cu") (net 6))
 (segment (start 142.933 78.566) (end 143.708 79.341) (width 0.15) (layer "F.Cu") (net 6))
 (segment (start 131.807264 78.566) (end 142.933 78.566) (width 0.15) (layer "F.Cu") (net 6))
 (segment (start 126.9575 79.366) (end 131.007264 79.366) (width 0.15) (layer "F.Cu") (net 6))
 (segment (start 111.833 80.616) (end 111.833 80.016) (width 0.15) (layer "F.Cu") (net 6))
 (via (at 143.683 82.466) (size 0.6) (drill 0.3) (layers "F.Cu" "B.Cu") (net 6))
 (via (at 126.683 79.0915) (size 0.6) (drill 0.3) (layers "F.Cu" "B.Cu") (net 6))
 (segment (start 143.683 82.466) (end 143.708 82.491) (width 0.15) (layer "B.Cu") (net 6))
 (segment (start 111.833 84.416) (end 111.833 80.016) (width 0.15) (layer "B.Cu") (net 6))
 (segment (start 126.1575 78.566) (end 126.683 79.0915) (width 0.15) (layer "B.Cu") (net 6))
 (segment (start 113.283 78.566) (end 126.1575 78.566) (width 0.15) (layer "B.Cu") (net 6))
 (segment (start 143.708 82.491) (end 143.708 84.616) (width 0.15) (layer "B.Cu") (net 6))
 (segment (start 111.833 80.016) (end 113.283 78.566) (width 0.15) (layer "B.Cu") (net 6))
 (segment (start 126.683 79.0915) (end 126.683 81.416) (width 0.15) (layer "B.Cu") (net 6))
 (segment (start 112.333 85.016) (end 112.333 83.916) (width 0.15) (layer "F.Cu") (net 7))
 (segment (start 142.458 82.441) (end 142.483 82.466) (width 0.15) (layer "F.Cu") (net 7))
 (segment (start 113.533 86.216) (end 112.333 85.016) (width 0.15) (layer "F.Cu") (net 7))
 (segment (start 124.483 85.5905) (end 123.8575 86.216) (width 0.15) (layer "F.Cu") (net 7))
 (segment (start 123.8575 86.216) (end 113.533 86.216) (width 0.15) (layer "F.Cu") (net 7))
 (segment (start 142.458 80.416) (end 142.458 82.441) (width 0.15) (layer "F.Cu") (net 7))
 (segment (start 124.483 83.616) (end 124.483 85.5905) (width 0.15) (layer "F.Cu") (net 7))
 (via (at 124.483 85.5905) (size 0.6) (drill 0.3) (layers "F.Cu" "B.Cu") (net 7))
 (via (at 142.483 82.466) (size 0.6) (drill 0.3) (layers "F.Cu" "B.Cu") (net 7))
 (segment (start 124.483 85.5905) (end 124.7075 85.366) (width 0.15) (layer "B.Cu") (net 7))
 (segment (start 142.483 82.466) (end 142.458 82.491) (width 0.15) (layer "B.Cu") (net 7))
 (segment (start 141.983 86.216) (end 142.458 85.741) (width 0.15) (layer "B.Cu") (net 7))
 (segment (start 113.533 86.216) (end 112.333 85.016) (width 0.15) (layer "B.Cu") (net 7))
 (segment (start 142.458 85.741) (end 142.458 84.616) (width 0.15) (layer "B.Cu") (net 7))
 (segment (start 112.333 85.016) (end 112.333 81.116) (width 0.15) (layer "B.Cu") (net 7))
 (segment (start 131.273991 85.366) (end 132.123991 86.216) (width 0.15) (layer "B.Cu") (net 7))
 (segment (start 124.7075 85.366) (end 131.273991 85.366) (width 0.15) (layer "B.Cu") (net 7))
 (segment (start 123.8575 86.216) (end 113.533 86.216) (width 0.15) (layer "B.Cu") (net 7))
 (segment (start 142.458 82.491) (end 142.458 84.616) (width 0.15) (layer "B.Cu") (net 7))
 (segment (start 132.123991 86.216) (end 141.983 86.216) (width 0.15) (layer "B.Cu") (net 7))
 (segment (start 124.483 85.5905) (end 123.8575 86.216) (width 0.15) (layer "B.Cu") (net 7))
 (segment (start 131.931528 78.866) (end 140.733 78.866) (width 0.15) (layer "F.Cu") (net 8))
 (segment (start 131.131528 79.666) (end 131.931528 78.866) (width 0.15) (layer "F.Cu") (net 8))
 (segment (start 141.208 79.341) (end 141.208 80.416) (width 0.15) (layer "F.Cu") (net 8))
 (segment (start 141.208 80.416) (end 141.208 82.391) (width 0.15) (layer "F.Cu") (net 8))
 (segment (start 113.983 78.866) (end 123.9575 78.866) (width 0.15) (layer "F.Cu") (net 8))
 (segment (start 124.7575 79.666) (end 131.131528 79.666) (width 0.15) (layer "F.Cu") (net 8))
 (segment (start 112.833 80.616) (end 112.833 80.016) (width 0.15) (layer "F.Cu") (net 8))
 (segment (start 123.9575 78.866) (end 124.483 79.3915) (width 0.15) (layer "F.Cu") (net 8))
 (segment (start 124.483 79.3915) (end 124.7575 79.666) (width 0.15) (layer "F.Cu") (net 8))
 (segment (start 140.733 78.866) (end 141.208 79.341) (width 0.15) (layer "F.Cu") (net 8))
 (segment (start 112.833 80.016) (end 113.983 78.866) (width 0.15) (layer "F.Cu") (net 8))
 (segment (start 141.208 82.391) (end 141.133 82.466) (width 0.15) (layer "F.Cu") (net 8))
 (via (at 141.133 82.466) (size 0.6) (drill 0.3) (layers "F.Cu" "B.Cu") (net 8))
 (via (at 124.483 79.3915) (size 0.6) (drill 0.3) (layers "F.Cu" "B.Cu") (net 8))
 (segment (start 113.983 78.866) (end 123.9575 78.866) (width 0.15) (layer "B.Cu") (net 8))
 (segment (start 141.208 82.541) (end 141.208 84.616) (width 0.15) (layer "B.Cu") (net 8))
 (segment (start 112.833 84.416) (end 112.833 80.016) (width 0.15) (layer "B.Cu") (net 8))
 (segment (start 123.9575 78.866) (end 124.483 79.3915) (width 0.15) (layer "B.Cu") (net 8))
 (segment (start 124.483 81.416) (end 124.483 79.3915) (width 0.15) (layer "B.Cu") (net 8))
 (segment (start 141.133 82.466) (end 141.208 82.541) (width 0.15) (layer "B.Cu") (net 8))
 (segment (start 112.833 80.016) (end 113.983 78.866) (width 0.15) (layer "B.Cu") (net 8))
 (segment (start 122.283 85.2905) (end 121.6575 85.916) (width 0.15) (layer "F.Cu") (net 9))
 (segment (start 122.283 83.616) (end 122.283 85.2905) (width 0.15) (layer "F.Cu") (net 9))
 (segment (start 114.233 85.916) (end 113.333 85.016) (width 0.15) (layer "F.Cu") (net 9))
 (segment (start 139.958 80.416) (end 139.958 82.441) (width 0.15) (layer "F.Cu") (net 9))
 (segment (start 113.333 85.016) (end 113.333 84.416) (width 0.15) (layer "F.Cu") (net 9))
 (segment (start 139.958 82.441) (end 139.933 82.466) (width 0.15) (layer "F.Cu") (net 9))
 (segment (start 121.6575 85.916) (end 114.233 85.916) (width 0.15) (layer "F.Cu") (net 9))
 (via (at 122.283 85.2905) (size 0.6) (drill 0.3) (layers "F.Cu" "B.Cu") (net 9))
 (via (at 139.933 82.466) (size 0.6) (drill 0.3) (layers "F.Cu" "B.Cu") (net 9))
 (segment (start 139.958 85.691) (end 139.958 84.616) (width 0.15) (layer "B.Cu") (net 9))
 (segment (start 131.398255 85.066) (end 132.248255 85.916) (width 0.15) (layer "B.Cu") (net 9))
 (segment (start 139.958 82.491) (end 139.958 84.616) (width 0.15) (layer "B.Cu") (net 9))
 (segment (start 122.283 85.2905) (end 121.6575 85.916) (width 0.15) (layer "B.Cu") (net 9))
 (segment (start 139.733 85.916) (end 139.958 85.691) (width 0.15) (layer "B.Cu") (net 9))
 (segment (start 139.933 82.466) (end 139.958 82.491) (width 0.15) (layer "B.Cu") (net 9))
 (segment (start 132.248255 85.916) (end 139.733 85.916) (width 0.15) (layer "B.Cu") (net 9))
 (segment (start 122.283 85.2905) (end 122.5075 85.066) (width 0.15) (layer "B.Cu") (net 9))
 (segment (start 114.233 85.916) (end 113.333 85.016) (width 0.15) (layer "B.Cu") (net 9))
 (segment (start 113.333 85.016) (end 113.333 80.616) (width 0.15) (layer "B.Cu") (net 9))
 (segment (start 121.6575 85.916) (end 114.233 85.916) (width 0.15) (layer "B.Cu") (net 9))
 (segment (start 122.5075 85.066) (end 131.398255 85.066) (width 0.15) (layer "B.Cu") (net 9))
 (segment (start 138.708 82.341) (end 138.583 82.466) (width 0.15) (layer "F.Cu") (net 10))
 (segment (start 138.533 79.166) (end 138.708 79.341) (width 0.15) (layer "F.Cu") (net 10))
 (segment (start 113.833 80.616) (end 113.833 80.016) (width 0.15) (layer "F.Cu") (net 10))
 (segment (start 113.833 80.016) (end 114.683 79.166) (width 0.15) (layer "F.Cu") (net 10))
 (segment (start 114.683 79.166) (end 121.7575 79.166) (width 0.15) (layer "F.Cu") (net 10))
 (segment (start 132.055792 79.166) (end 138.533 79.166) (width 0.15) (layer "F.Cu") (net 10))
 (segment (start 122.5575 79.966) (end 131.255792 79.966) (width 0.15) (layer "F.Cu") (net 10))
 (segment (start 121.7575 79.166) (end 122.283 79.6915) (width 0.15) (layer "F.Cu") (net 10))
 (segment (start 138.708 79.341) (end 138.708 80.416) (width 0.15) (layer "F.Cu") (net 10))
 (segment (start 122.283 79.6915) (end 122.5575 79.966) (width 0.15) (layer "F.Cu") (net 10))
 (segment (start 131.255792 79.966) (end 132.055792 79.166) (width 0.15) (layer "F.Cu") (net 10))
 (segment (start 138.708 80.416) (end 138.708 82.341) (width 0.15) (layer "F.Cu") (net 10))
 (via (at 138.583 82.466) (size 0.6) (drill 0.3) (layers "F.Cu" "B.Cu") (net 10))
 (via (at 122.283 79.6915) (size 0.6) (drill 0.3) (layers "F.Cu" "B.Cu") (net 10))
 (segment (start 122.283 79.6915) (end 122.283 81.416) (width 0.15) (layer "B.Cu") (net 10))
 (segment (start 114.683 79.166) (end 121.7575 79.166) (width 0.15) (layer "B.Cu") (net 10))
 (segment (start 138.583 82.466) (end 138.708 82.591) (width 0.15) (layer "B.Cu") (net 10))
 (segment (start 121.7575 79.166) (end 122.283 79.6915) (width 0.15) (layer "B.Cu") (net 10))
 (segment (start 113.833 84.416) (end 113.833 80.016) (width 0.15) (layer "B.Cu") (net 10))
 (segment (start 113.833 80.016) (end 114.683 79.166) (width 0.15) (layer "B.Cu") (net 10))
 (segment (start 138.708 82.591) (end 138.708 84.616) (width 0.15) (layer "B.Cu") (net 10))
 (segment (start 114.933 85.616) (end 119.483 85.616) (width 0.15) (layer "F.Cu") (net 11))
 (segment (start 120.083 85.016) (end 120.083 83.616) (width 0.15) (layer "F.Cu") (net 11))
 (segment (start 137.458 82.391) (end 137.383 82.466) (width 0.15) (layer "F.Cu") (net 11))
 (segment (start 114.333 84.416) (end 114.333 85.016) (width 0.15) (layer "F.Cu") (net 11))
 (segment (start 137.458 80.416) (end 137.458 82.391) (width 0.15) (layer "F.Cu") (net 11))
 (segment (start 114.333 85.016) (end 114.933 85.616) (width 0.15) (layer "F.Cu") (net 11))
 (segment (start 119.483 85.616) (end 120.083 85.016) (width 0.15) (layer "F.Cu") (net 11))
 (via (at 137.383 82.466) (size 0.6) (drill 0.3) (layers "F.Cu" "B.Cu") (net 11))
 (segment (start 137.458 82.541) (end 137.458 84.616) (width 0.15) (layer "B.Cu") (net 11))
 (segment (start 114.933 85.616) (end 119.483 85.616) (width 0.15) (layer "B.Cu") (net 11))
 (segment (start 137.383 82.466) (end 137.458 82.541) (width 0.15) (layer "B.Cu") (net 11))
 (segment (start 121.233 84.766) (end 120.083 83.616) (width 0.15) (layer "B.Cu") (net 11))
 (segment (start 120.083 85.016) (end 120.083 83.616) (width 0.15) (layer "B.Cu") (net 11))
 (segment (start 135.733 81.866) (end 132.833 84.766) (width 0.15) (layer "B.Cu") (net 11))
 (segment (start 136.783 81.866) (end 135.733 81.866) (width 0.15) (layer "B.Cu") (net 11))
 (segment (start 114.333 85.016) (end 114.933 85.616) (width 0.15) (layer "B.Cu") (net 11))
 (segment (start 119.483 85.616) (end 120.083 85.016) (width 0.15) (layer "B.Cu") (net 11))
 (segment (start 114.333 80.616) (end 114.333 85.016) (width 0.15) (layer "B.Cu") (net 11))
 (segment (start 137.383 82.466) (end 136.783 81.866) (width 0.15) (layer "B.Cu") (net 11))
 (segment (start 132.833 84.766) (end 121.233 84.766) (width 0.15) (layer "B.Cu") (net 11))
 (segment (start 119.583 79.466) (end 120.083 79.966) (width 0.15) (layer "F.Cu") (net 12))
 (segment (start 131.380056 80.266) (end 121.233 80.266) (width 0.15) (layer "F.Cu") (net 12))
 (segment (start 115.383 79.466) (end 119.583 79.466) (width 0.15) (layer "F.Cu") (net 12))
 (segment (start 136.208 79.466) (end 132.180056 79.466) (width 0.15) (layer "F.Cu") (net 12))
 (segment (start 114.833 80.616) (end 114.833 80.016) (width 0.15) (layer "F.Cu") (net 12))
 (segment (start 121.233 80.266) (end 120.083 81.416) (width 0.15) (layer "F.Cu") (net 12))
 (segment (start 136.208 82.441) (end 136.183 82.466) (width 0.15) (layer "F.Cu") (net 12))
 (segment (start 136.208 80.416) (end 136.208 79.466) (width 0.15) (layer "F.Cu") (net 12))
 (segment (start 120.083 79.966) (end 120.083 81.416) (width 0.15) (layer "F.Cu") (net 12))
 (segment (start 132.180056 79.466) (end 131.380056 80.266) (width 0.15) (layer "F.Cu") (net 12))
 (segment (start 114.833 80.016) (end 115.383 79.466) (width 0.15) (layer "F.Cu") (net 12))
 (segment (start 136.208 80.416) (end 136.208 82.441) (width 0.15) (layer "F.Cu") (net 12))
 (via (at 136.183 82.466) (size 0.6) (drill 0.3) (layers "F.Cu" "B.Cu") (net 12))
 (segment (start 114.833 80.016) (end 115.383 79.466) (width 0.15) (layer "B.Cu") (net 12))
 (segment (start 120.083 79.966) (end 120.083 81.416) (width 0.15) (layer "B.Cu") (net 12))
 (segment (start 119.583 79.466) (end 120.083 79.966) (width 0.15) (layer "B.Cu") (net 12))
 (segment (start 136.208 82.491) (end 136.208 84.616) (width 0.15) (layer "B.Cu") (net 12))
 (segment (start 115.383 79.466) (end 119.583 79.466) (width 0.15) (layer "B.Cu") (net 12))
 (segment (start 136.183 82.466) (end 136.208 82.491) (width 0.15) (layer "B.Cu") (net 12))
 (segment (start 114.833 84.416) (end 114.833 80.016) (width 0.15) (layer "B.Cu") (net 12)))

